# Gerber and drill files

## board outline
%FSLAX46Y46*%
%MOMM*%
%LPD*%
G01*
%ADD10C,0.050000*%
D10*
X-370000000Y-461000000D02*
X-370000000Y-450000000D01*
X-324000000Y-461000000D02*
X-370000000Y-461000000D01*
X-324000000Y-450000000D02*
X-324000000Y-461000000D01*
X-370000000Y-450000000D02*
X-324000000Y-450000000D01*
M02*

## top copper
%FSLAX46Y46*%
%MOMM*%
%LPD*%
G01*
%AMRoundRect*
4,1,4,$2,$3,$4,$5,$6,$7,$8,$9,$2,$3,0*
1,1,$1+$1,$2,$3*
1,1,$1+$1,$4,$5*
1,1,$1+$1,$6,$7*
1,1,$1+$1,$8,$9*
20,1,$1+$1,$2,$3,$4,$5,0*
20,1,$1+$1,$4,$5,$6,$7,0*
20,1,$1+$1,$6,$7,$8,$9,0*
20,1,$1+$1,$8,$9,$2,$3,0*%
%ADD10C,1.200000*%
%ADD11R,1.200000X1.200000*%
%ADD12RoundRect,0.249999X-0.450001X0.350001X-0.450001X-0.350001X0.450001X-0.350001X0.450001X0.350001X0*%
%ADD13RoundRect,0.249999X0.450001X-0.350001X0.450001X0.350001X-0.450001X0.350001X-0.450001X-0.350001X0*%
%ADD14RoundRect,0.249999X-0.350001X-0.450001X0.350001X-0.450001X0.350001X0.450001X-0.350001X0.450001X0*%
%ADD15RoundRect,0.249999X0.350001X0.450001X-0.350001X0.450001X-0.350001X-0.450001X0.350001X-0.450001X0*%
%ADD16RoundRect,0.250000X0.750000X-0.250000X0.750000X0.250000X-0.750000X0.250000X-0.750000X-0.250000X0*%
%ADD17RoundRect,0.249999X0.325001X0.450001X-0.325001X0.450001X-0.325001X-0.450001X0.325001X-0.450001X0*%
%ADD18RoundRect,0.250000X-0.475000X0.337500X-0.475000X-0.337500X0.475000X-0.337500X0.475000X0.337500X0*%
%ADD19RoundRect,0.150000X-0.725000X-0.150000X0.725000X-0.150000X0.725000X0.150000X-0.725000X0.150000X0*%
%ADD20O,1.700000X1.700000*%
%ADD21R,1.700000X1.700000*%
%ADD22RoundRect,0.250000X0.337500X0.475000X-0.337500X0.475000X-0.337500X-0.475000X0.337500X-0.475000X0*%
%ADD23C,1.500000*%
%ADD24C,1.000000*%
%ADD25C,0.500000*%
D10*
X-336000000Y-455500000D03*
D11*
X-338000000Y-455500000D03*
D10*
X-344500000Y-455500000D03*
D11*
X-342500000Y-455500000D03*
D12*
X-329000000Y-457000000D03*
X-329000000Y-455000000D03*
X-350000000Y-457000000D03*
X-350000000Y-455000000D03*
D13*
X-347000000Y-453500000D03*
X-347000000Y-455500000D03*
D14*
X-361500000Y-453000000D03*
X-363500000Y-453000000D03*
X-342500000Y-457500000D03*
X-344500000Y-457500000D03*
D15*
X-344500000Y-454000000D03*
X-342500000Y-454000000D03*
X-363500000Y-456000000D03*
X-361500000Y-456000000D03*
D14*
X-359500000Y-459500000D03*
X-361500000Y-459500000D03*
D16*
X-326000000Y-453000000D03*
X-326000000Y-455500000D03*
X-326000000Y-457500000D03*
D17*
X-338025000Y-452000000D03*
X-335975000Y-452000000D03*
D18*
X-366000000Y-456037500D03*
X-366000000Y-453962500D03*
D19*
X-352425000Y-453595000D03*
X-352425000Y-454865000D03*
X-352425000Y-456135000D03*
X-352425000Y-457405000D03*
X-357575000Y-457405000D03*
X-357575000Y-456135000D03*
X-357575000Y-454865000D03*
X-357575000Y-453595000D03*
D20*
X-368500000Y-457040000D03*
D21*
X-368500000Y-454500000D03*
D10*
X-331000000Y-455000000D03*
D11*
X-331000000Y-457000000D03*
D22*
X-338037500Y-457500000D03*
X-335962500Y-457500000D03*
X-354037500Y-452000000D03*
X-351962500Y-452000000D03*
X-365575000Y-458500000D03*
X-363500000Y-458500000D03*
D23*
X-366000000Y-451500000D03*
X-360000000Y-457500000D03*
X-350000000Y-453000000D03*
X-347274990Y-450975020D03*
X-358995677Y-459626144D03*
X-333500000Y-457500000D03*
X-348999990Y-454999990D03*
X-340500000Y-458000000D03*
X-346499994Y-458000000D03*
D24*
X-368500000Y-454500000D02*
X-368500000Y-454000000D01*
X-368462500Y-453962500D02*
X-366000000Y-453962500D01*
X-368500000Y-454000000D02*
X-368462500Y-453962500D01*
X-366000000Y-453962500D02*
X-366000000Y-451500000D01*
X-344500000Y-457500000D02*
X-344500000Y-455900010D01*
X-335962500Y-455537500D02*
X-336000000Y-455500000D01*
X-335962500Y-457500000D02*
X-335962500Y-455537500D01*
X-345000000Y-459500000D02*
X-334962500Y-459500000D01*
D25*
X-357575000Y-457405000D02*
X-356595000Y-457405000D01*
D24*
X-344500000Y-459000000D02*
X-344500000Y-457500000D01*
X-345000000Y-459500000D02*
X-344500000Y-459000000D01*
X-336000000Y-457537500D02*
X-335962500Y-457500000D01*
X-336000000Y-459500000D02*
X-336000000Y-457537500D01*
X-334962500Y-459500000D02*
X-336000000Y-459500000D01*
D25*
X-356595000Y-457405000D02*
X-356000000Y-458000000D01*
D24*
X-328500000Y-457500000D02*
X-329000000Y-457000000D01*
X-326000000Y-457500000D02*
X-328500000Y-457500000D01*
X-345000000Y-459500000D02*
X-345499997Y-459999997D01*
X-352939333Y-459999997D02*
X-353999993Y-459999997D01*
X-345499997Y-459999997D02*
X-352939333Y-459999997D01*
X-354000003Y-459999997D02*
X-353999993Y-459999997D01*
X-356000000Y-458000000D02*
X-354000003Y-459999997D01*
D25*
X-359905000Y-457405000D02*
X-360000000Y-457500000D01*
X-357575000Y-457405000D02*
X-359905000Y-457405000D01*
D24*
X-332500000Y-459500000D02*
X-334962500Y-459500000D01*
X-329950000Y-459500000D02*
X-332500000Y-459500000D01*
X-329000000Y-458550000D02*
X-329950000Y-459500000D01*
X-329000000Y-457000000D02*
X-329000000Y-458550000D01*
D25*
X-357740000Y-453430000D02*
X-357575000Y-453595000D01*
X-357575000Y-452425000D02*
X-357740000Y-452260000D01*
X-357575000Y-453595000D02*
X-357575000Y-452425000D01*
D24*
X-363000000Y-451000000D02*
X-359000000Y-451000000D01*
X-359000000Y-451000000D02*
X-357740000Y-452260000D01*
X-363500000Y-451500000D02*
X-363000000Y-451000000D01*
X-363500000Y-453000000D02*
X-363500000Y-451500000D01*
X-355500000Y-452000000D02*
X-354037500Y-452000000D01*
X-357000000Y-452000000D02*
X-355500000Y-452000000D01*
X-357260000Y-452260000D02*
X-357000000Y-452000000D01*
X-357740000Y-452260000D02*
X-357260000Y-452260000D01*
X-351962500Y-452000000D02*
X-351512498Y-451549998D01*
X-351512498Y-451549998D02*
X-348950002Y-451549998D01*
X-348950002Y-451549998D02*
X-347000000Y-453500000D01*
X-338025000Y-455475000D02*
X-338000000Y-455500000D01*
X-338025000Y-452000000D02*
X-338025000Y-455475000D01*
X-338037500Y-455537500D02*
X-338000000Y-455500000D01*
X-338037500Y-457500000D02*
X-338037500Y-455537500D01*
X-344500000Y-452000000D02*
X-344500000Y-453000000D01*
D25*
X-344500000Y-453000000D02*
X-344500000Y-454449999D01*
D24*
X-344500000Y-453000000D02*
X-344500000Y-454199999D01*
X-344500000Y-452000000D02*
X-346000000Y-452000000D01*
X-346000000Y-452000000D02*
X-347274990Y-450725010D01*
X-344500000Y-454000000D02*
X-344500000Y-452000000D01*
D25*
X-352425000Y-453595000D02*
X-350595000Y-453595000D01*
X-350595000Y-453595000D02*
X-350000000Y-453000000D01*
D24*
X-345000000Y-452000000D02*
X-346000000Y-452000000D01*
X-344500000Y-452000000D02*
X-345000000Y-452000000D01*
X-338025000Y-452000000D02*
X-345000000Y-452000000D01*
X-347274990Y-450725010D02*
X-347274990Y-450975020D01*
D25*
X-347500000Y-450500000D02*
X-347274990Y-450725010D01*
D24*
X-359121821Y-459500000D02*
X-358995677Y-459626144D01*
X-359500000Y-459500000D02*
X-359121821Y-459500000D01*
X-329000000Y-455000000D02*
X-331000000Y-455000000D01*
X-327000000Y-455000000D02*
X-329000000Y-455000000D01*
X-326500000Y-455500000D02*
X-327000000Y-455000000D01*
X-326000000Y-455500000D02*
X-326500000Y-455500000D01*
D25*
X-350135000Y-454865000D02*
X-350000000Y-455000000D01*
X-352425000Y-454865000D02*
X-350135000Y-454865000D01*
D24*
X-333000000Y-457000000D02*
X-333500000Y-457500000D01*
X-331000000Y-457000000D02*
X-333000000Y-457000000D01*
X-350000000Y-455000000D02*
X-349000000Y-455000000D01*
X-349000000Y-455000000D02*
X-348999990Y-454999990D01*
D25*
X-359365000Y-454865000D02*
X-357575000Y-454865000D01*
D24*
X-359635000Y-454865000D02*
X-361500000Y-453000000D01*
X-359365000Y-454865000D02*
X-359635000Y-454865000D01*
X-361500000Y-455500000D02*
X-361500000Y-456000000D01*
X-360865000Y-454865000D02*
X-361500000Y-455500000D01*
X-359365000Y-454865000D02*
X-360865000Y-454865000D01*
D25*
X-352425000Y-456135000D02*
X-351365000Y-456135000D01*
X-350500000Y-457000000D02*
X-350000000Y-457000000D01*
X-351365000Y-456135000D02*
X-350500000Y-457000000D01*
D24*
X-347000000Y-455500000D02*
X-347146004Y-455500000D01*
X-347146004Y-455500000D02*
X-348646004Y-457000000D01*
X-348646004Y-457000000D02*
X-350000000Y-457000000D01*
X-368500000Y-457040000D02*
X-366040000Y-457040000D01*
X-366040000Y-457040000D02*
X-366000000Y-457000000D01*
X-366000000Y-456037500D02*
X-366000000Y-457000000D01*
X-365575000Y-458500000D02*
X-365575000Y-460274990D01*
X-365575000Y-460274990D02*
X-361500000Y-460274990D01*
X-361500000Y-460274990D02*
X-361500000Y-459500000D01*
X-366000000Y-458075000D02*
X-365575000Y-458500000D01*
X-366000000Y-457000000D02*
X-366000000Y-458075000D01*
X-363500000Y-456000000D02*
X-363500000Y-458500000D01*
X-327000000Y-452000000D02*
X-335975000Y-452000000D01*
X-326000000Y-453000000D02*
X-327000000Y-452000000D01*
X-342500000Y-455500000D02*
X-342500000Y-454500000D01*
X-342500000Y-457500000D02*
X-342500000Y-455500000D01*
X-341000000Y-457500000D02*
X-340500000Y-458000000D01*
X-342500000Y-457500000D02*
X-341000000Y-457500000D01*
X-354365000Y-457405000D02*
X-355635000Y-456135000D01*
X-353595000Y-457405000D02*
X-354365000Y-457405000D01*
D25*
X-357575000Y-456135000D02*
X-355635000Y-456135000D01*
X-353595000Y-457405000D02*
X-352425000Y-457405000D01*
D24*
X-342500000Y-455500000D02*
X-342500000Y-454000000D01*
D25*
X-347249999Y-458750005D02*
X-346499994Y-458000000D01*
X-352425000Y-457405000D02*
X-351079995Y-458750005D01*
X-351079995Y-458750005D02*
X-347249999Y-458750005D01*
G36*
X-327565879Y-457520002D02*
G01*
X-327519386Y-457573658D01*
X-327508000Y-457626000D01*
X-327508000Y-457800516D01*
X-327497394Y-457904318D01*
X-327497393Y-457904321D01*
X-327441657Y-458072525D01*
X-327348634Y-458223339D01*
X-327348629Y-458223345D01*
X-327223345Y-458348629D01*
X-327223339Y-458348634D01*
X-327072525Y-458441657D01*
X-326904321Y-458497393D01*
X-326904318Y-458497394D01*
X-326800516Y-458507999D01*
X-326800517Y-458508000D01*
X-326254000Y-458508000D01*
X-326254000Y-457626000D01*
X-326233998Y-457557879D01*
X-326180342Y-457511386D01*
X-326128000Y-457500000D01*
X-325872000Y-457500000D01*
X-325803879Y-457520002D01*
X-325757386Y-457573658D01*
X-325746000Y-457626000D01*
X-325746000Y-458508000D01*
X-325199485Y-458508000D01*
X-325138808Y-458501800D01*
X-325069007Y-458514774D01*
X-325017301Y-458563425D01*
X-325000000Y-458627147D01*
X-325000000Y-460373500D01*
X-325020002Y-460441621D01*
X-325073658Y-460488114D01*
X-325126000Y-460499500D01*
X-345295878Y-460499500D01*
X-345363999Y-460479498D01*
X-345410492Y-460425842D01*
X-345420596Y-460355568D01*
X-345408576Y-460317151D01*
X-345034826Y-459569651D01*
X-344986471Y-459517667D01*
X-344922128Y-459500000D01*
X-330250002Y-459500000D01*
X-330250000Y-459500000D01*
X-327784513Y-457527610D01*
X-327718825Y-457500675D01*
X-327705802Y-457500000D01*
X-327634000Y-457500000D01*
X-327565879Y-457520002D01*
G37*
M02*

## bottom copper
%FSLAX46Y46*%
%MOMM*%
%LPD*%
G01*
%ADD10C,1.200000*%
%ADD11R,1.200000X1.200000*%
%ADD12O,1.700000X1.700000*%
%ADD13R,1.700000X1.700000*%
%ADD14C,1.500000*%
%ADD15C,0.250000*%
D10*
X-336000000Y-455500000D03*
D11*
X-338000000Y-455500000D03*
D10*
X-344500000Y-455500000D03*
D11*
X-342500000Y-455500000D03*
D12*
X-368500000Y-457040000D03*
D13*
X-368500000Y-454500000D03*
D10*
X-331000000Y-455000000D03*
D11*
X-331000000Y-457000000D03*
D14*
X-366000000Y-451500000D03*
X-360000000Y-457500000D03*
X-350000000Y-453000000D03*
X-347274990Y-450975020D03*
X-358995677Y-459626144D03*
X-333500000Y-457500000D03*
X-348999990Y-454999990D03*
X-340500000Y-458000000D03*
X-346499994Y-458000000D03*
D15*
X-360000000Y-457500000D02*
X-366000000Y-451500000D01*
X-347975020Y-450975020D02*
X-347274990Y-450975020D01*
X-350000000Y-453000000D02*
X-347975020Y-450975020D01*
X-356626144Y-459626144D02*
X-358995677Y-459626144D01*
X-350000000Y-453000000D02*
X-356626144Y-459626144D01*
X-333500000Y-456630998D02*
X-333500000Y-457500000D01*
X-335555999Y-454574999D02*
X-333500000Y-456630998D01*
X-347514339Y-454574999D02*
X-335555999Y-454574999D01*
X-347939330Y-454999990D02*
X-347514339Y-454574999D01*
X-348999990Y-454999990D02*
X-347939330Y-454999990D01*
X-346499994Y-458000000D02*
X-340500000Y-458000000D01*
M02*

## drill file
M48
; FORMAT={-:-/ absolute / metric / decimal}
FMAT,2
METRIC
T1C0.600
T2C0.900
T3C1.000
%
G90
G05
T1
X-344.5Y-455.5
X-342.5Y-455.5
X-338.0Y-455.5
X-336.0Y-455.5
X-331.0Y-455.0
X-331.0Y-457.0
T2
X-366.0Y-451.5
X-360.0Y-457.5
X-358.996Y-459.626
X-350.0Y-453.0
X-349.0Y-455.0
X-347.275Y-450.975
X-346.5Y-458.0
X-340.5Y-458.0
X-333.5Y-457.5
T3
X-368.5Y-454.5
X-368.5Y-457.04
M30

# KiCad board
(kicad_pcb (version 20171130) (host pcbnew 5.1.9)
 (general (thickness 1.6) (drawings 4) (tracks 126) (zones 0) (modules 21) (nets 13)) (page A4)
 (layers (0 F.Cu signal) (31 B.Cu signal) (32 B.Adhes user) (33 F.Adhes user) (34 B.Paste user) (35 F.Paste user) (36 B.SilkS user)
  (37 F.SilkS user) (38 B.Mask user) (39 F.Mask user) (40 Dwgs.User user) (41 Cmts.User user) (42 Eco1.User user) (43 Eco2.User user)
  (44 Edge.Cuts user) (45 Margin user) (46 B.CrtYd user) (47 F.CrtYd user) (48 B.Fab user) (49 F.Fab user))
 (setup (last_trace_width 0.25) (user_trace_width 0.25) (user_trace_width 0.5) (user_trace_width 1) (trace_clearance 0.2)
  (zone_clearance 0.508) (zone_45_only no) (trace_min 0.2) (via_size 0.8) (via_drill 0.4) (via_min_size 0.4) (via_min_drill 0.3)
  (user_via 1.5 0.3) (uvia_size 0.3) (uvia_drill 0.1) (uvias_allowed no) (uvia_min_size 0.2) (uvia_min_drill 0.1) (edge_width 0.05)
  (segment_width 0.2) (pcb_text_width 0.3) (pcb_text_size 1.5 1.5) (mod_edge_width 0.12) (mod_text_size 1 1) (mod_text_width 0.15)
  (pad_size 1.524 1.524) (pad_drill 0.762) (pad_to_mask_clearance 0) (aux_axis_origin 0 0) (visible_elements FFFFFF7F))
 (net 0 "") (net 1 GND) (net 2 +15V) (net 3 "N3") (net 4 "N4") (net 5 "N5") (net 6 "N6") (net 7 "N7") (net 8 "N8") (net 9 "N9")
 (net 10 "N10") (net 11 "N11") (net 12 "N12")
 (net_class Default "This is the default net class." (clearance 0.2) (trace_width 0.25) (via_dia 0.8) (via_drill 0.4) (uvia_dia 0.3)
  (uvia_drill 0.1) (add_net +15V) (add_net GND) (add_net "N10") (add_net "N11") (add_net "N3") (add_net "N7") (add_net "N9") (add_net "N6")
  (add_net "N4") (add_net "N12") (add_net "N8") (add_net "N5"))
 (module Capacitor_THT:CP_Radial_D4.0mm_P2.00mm (layer B.Cu) (at -338 455.5)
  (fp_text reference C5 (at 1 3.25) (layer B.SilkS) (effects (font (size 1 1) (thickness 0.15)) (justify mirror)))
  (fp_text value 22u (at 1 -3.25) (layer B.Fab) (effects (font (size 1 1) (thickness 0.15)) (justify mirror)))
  (pad 2 thru_hole circle (at 2 0) (size 1.2 1.2) (drill 0.6) (layers *.Cu *.Mask) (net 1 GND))
  (pad 1 thru_hole rect (at 0 0) (size 1.2 1.2) (drill 0.6) (layers *.Cu *.Mask) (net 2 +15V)))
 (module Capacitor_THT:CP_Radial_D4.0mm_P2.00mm (layer B.Cu) (at -342.5 455.5 180)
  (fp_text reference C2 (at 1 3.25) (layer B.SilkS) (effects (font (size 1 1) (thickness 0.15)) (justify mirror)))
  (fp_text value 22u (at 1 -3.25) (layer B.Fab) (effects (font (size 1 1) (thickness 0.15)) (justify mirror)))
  (pad 2 thru_hole circle (at 2 0 180) (size 1.2 1.2) (drill 0.6) (layers *.Cu *.Mask) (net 1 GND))
  (pad 1 thru_hole rect (at 0 0 180) (size 1.2 1.2) (drill 0.6) (layers *.Cu *.Mask) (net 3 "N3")))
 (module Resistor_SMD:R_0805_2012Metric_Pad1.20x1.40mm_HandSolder (layer F.Cu) (at -329 456 270)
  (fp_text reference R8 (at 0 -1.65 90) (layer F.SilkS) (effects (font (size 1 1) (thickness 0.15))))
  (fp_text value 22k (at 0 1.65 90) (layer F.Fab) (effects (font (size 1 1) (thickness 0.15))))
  (pad 2 smd roundrect (at 1 0 270) (size 1.2 1.4) (layers F.Cu F.Paste F.Mask) (roundrect_rratio 0.2083325) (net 1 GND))
  (pad 1 smd roundrect (at -1 0 270) (size 1.2 1.4) (layers F.Cu F.Paste F.Mask) (roundrect_rratio 0.2083325) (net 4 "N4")))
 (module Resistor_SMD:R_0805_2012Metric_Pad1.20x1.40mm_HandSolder (layer F.Cu) (at -350 456 270)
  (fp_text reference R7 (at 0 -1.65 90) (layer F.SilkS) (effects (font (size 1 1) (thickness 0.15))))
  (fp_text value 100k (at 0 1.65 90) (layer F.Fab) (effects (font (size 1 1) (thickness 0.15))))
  (pad 2 smd roundrect (at 1 0 270) (size 1.2 1.4) (layers F.Cu F.Paste F.Mask) (roundrect_rratio 0.2083325) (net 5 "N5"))
  (pad 1 smd roundrect (at -1 0 270) (size 1.2 1.4) (layers F.Cu F.Paste F.Mask) (roundrect_rratio 0.2083325) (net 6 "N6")))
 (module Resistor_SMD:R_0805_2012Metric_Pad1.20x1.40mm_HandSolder (layer F.Cu) (at -347 454.5 90)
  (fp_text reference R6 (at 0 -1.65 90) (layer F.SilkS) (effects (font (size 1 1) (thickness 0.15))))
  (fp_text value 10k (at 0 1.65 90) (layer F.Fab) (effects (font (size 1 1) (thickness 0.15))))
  (pad 2 smd roundrect (at 1 0 90) (size 1.2 1.4) (layers F.Cu F.Paste F.Mask) (roundrect_rratio 0.2083325) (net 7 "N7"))
  (pad 1 smd roundrect (at -1 0 90) (size 1.2 1.4) (layers F.Cu F.Paste F.Mask) (roundrect_rratio 0.2083325) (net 5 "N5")))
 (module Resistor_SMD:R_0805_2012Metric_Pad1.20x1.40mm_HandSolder (layer F.Cu) (at -362.5 453)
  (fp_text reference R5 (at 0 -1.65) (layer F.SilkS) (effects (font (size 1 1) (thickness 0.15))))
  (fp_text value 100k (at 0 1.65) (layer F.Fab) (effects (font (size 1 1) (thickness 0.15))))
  (pad 2 smd roundrect (at 1 0) (size 1.2 1.4) (layers F.Cu F.Paste F.Mask) (roundrect_rratio 0.2083325) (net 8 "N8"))
  (pad 1 smd roundrect (at -1 0) (size 1.2 1.4) (layers F.Cu F.Paste F.Mask) (roundrect_rratio 0.2083325) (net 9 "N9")))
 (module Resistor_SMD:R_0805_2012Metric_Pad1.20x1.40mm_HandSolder (layer F.Cu) (at -343.5 457.5)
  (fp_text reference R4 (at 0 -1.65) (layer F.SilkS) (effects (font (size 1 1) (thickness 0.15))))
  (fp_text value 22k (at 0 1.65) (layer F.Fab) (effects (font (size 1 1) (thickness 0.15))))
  (pad 2 smd roundrect (at 1 0) (size 1.2 1.4) (layers F.Cu F.Paste F.Mask) (roundrect_rratio 0.2083325) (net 3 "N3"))
  (pad 1 smd roundrect (at -1 0) (size 1.2 1.4) (layers F.Cu F.Paste F.Mask) (roundrect_rratio 0.2083325) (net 1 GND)))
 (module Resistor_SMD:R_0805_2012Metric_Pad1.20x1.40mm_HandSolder (layer F.Cu) (at -343.5 454 180)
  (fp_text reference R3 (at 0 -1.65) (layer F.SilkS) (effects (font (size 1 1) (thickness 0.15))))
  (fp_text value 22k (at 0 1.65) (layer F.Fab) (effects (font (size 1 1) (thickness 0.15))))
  (pad 2 smd roundrect (at 1 0 180) (size 1.2 1.4) (layers F.Cu F.Paste F.Mask) (roundrect_rratio 0.2083325) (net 2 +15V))
  (pad 1 smd roundrect (at -1 0 180) (size 1.2 1.4) (layers F.Cu F.Paste F.Mask) (roundrect_rratio 0.2083325) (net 3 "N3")))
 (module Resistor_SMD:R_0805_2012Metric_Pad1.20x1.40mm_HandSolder (layer F.Cu) (at -362.5 456 180)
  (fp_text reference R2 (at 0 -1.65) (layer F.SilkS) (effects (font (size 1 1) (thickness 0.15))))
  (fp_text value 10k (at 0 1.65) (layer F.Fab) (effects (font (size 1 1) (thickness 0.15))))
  (pad 2 smd roundrect (at 1 0 180) (size 1.2 1.4) (layers F.Cu F.Paste F.Mask) (roundrect_rratio 0.2083325) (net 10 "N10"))
  (pad 1 smd roundrect (at -1 0 180) (size 1.2 1.4) (layers F.Cu F.Paste F.Mask) (roundrect_rratio 0.2083325) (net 8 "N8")))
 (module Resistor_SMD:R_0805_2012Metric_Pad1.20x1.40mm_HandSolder (layer F.Cu) (at -360.5 459.5)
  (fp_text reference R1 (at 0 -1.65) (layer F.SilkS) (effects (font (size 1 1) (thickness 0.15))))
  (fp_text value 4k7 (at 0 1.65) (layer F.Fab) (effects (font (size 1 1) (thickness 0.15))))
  (pad 2 smd roundrect (at 1 0) (size 1.2 1.4) (layers F.Cu F.Paste F.Mask) (roundrect_rratio 0.2083325) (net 2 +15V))
  (pad 1 smd roundrect (at -1 0) (size 1.2 1.4) (layers F.Cu F.Paste F.Mask) (roundrect_rratio 0.2083325) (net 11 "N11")))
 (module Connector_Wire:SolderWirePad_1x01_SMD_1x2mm (layer F.Cu) (at -326 453 90)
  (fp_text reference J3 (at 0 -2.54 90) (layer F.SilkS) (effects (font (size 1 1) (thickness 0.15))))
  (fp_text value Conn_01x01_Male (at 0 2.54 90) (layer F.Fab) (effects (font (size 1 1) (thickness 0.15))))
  (pad 1 smd roundrect (at 0 0 90) (size 1 2) (layers F.Cu F.Paste F.Mask) (roundrect_rratio 0.25) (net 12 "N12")))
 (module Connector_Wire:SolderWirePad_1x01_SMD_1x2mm (layer F.Cu) (at -326 455.5 90)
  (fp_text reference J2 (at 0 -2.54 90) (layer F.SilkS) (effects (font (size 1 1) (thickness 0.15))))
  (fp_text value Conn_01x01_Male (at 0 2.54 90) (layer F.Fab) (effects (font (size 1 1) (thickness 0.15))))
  (pad 1 smd roundrect (at 0 0 90) (size 1 2) (layers F.Cu F.Paste F.Mask) (roundrect_rratio 0.25) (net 4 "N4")))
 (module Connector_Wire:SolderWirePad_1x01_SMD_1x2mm (layer F.Cu) (at -326 457.5 90)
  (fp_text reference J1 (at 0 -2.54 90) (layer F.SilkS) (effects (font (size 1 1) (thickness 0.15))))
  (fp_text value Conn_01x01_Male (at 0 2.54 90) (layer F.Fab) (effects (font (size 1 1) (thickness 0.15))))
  (pad 1 smd roundrect (at 0 0 90) (size 1 2) (layers F.Cu F.Paste F.Mask) (roundrect_rratio 0.25) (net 1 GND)))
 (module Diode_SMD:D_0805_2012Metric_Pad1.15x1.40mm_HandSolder (layer F.Cu) (at -337 452 180)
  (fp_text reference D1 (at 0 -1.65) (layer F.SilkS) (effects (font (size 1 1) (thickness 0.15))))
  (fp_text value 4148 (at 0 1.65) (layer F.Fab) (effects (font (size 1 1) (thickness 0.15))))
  (pad 2 smd roundrect (at 1.025 0 180) (size 1.15 1.4) (layers F.Cu F.Paste F.Mask) (roundrect_rratio 0.2173904347826087) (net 2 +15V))
  (pad 1 smd roundrect (at -1.025 0 180) (size 1.15 1.4) (layers F.Cu F.Paste F.Mask) (roundrect_rratio 0.2173904347826087) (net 12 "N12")))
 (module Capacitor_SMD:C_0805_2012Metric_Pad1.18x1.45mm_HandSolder (layer F.Cu) (at -366 455 270)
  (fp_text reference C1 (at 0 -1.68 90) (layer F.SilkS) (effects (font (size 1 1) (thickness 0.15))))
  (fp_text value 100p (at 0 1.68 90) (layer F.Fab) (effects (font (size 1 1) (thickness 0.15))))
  (pad 2 smd roundrect (at 1.0375 0 270) (size 1.175 1.45) (layers F.Cu F.Paste F.Mask) (roundrect_rratio 0.2127659574468085) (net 11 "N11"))
  (pad 1 smd roundrect (at -1.0375 0 270) (size 1.175 1.45) (layers F.Cu F.Paste F.Mask) (roundrect_rratio 0.2127659574468085) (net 1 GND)))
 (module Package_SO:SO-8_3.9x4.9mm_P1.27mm (layer F.Cu) (at -355 455.5)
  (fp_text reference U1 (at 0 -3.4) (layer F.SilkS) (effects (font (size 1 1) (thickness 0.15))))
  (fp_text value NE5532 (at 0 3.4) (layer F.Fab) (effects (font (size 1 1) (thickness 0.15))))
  (pad 8 smd roundrect (at 2.575 -1.905) (size 1.75 0.6) (layers F.Cu F.Paste F.Mask) (roundrect_rratio 0.25) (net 2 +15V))
  (pad 7 smd roundrect (at 2.575 -0.635) (size 1.75 0.6) (layers F.Cu F.Paste F.Mask) (roundrect_rratio 0.25) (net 6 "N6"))
  (pad 6 smd roundrect (at 2.575 0.635) (size 1.75 0.6) (layers F.Cu F.Paste F.Mask) (roundrect_rratio 0.25) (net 5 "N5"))
  (pad 5 smd roundrect (at 2.575 1.905) (size 1.75 0.6) (layers F.Cu F.Paste F.Mask) (roundrect_rratio 0.25) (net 3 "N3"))
  (pad 4 smd roundrect (at -2.575 1.905) (size 1.75 0.6) (layers F.Cu F.Paste F.Mask) (roundrect_rratio 0.25) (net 1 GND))
  (pad 3 smd roundrect (at -2.575 0.635) (size 1.75 0.6) (layers F.Cu F.Paste F.Mask) (roundrect_rratio 0.25) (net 3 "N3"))
  (pad 2 smd roundrect (at -2.575 -0.635) (size 1.75 0.6) (layers F.Cu F.Paste F.Mask) (roundrect_rratio 0.25) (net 8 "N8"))
  (pad 1 smd roundrect (at -2.575 -1.905) (size 1.75 0.6) (layers F.Cu F.Paste F.Mask) (roundrect_rratio 0.25) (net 9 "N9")))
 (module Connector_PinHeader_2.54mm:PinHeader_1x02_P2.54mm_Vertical (layer B.Cu) (at -368.5 454.5 180)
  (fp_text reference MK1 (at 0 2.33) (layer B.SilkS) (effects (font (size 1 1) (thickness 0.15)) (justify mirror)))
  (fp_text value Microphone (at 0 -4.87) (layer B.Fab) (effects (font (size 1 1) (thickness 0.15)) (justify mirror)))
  (pad 2 thru_hole oval (at 0 -2.54 180) (size 1.7 1.7) (drill 1) (layers *.Cu *.Mask) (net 11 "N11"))
  (pad 1 thru_hole rect (at 0 0 180) (size 1.7 1.7) (drill 1) (layers *.Cu *.Mask) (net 1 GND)))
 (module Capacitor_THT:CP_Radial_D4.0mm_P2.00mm (layer B.Cu) (at -331 457 90)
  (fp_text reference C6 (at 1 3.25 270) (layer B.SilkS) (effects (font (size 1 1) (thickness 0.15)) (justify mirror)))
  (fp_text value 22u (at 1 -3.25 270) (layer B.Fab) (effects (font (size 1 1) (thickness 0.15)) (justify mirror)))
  (pad 2 thru_hole circle (at 2 0 90) (size 1.2 1.2) (drill 0.6) (layers *.Cu *.Mask) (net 4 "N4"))
  (pad 1 thru_hole rect (at 0 0 90) (size 1.2 1.2) (drill 0.6) (layers *.Cu *.Mask) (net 6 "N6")))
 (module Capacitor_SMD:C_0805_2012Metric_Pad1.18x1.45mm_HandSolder (layer F.Cu) (at -337 457.5 180)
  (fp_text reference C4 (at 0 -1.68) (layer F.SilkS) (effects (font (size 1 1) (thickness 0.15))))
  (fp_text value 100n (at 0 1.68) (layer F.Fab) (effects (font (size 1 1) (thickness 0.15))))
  (pad 2 smd roundrect (at 1.0375 0 180) (size 1.175 1.45) (layers F.Cu F.Paste F.Mask) (roundrect_rratio 0.2127659574468085) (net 2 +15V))
  (pad 1 smd roundrect (at -1.0375 0 180) (size 1.175 1.45) (layers F.Cu F.Paste F.Mask) (roundrect_rratio 0.2127659574468085) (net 1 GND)))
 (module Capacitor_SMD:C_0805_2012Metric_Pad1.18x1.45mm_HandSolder (layer F.Cu) (at -353 452 180)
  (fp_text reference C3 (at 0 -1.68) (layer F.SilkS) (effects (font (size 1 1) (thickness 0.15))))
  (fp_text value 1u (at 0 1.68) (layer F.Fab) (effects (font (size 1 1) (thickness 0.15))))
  (pad 2 smd roundrect (at 1.0375 0 180) (size 1.175 1.45) (layers F.Cu F.Paste F.Mask) (roundrect_rratio 0.2127659574468085) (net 9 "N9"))
  (pad 1 smd roundrect (at -1.0375 0 180) (size 1.175 1.45) (layers F.Cu F.Paste F.Mask) (roundrect_rratio 0.2127659574468085) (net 7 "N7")))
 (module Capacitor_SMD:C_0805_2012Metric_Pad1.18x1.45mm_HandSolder (layer F.Cu) (at -364.5375 458.5 180)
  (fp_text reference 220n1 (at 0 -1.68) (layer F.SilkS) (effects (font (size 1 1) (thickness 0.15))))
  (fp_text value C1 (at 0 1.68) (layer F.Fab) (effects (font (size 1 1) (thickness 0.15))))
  (pad 2 smd roundrect (at 1.0375 0 180) (size 1.175 1.45) (layers F.Cu F.Paste F.Mask) (roundrect_rratio 0.2127659574468085) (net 11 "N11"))
  (pad 1 smd roundrect (at -1.0375 0 180) (size 1.175 1.45) (layers F.Cu F.Paste F.Mask) (roundrect_rratio 0.2127659574468085)
   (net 10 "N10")))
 (gr_line (start -370 461) (end -370 450) (layer Edge.Cuts) (width 0.05))
 (gr_line (start -324 461) (end -370 461) (layer Edge.Cuts) (width 0.05))
 (gr_line (start -324 450) (end -324 461) (layer Edge.Cuts) (width 0.05))
 (gr_line (start -370 450) (end -324 450) (layer Edge.Cuts) (width 0.05))
 (segment (start -368.5 454.5) (end -368.5 454) (width 1) (layer F.Cu) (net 1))
 (segment (start -368.4625 453.9625) (end -366 453.9625) (width 1) (layer F.Cu) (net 1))
 (segment (start -368.5 454) (end -368.4625 453.9625) (width 1) (layer F.Cu) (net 1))
 (via (at -366 451.5) (size 1.5) (drill 0.9) (layers F.Cu B.Cu) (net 1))
 (segment (start -366 453.9625) (end -366 451.5) (width 1) (layer F.Cu) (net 1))
 (segment (start -344.5 457.5) (end -344.5 455.90001) (width 1) (layer F.Cu) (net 1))
 (segment (start -335.9625 455.5375) (end -336 455.5) (width 1) (layer F.Cu) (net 1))
 (segment (start -335.9625 457.5) (end -335.9625 455.5375) (width 1) (layer F.Cu) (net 1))
 (segment (start -345 459.5) (end -334.9625 459.5) (width 1) (layer F.Cu) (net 1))
 (segment (start -357.575 457.405) (end -356.595 457.405) (width 0.5) (layer F.Cu) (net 1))
 (segment (start -344.5 459) (end -344.5 457.5) (width 1) (layer F.Cu) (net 1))
 (segment (start -345 459.5) (end -344.5 459) (width 1) (layer F.Cu) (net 1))
 (segment (start -336 457.5375) (end -335.9625 457.5) (width 1) (layer F.Cu) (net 1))
 (segment (start -336 459.5) (end -336 457.5375) (width 1) (layer F.Cu) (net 1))
 (segment (start -334.9625 459.5) (end -336 459.5) (width 1) (layer F.Cu) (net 1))
 (segment (start -356.595 457.405) (end -356 458) (width 0.5) (layer F.Cu) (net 1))
 (segment (start -328.5 457.5) (end -329 457) (width 1) (layer F.Cu) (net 1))
 (segment (start -326 457.5) (end -328.5 457.5) (width 1) (layer F.Cu) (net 1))
 (segment (start -345 459.5) (end -345.499997 459.999997) (width 1) (layer F.Cu) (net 1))
 (segment (start -352.939333 459.999997) (end -353.999993 459.999997) (width 1) (layer F.Cu) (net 1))
 (segment (start -345.499997 459.999997) (end -352.939333 459.999997) (width 1) (layer F.Cu) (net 1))
 (segment (start -354.000003 459.999997) (end -353.999993 459.999997) (width 1) (layer F.Cu) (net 1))
 (segment (start -356 458) (end -354.000003 459.999997) (width 1) (layer F.Cu) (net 1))
 (via (at -360 457.5) (size 1.5) (drill 0.9) (layers F.Cu B.Cu) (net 1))
 (segment (start -359.905 457.405) (end -360 457.5) (width 0.5) (layer F.Cu) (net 1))
 (segment (start -357.575 457.405) (end -359.905 457.405) (width 0.5) (layer F.Cu) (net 1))
 (segment (start -360 457.5) (end -366 451.5) (width 0.25) (layer B.Cu) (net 1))
 (segment (start -332.5 459.5) (end -334.9625 459.5) (width 1) (layer F.Cu) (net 1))
 (segment (start -329.95 459.5) (end -332.5 459.5) (width 1) (layer F.Cu) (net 1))
 (segment (start -329 458.55) (end -329.95 459.5) (width 1) (layer F.Cu) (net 1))
 (segment (start -329 457) (end -329 458.55) (width 1) (layer F.Cu) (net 1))
 (segment (start -357.74 453.43) (end -357.575 453.595) (width 0.5) (layer F.Cu) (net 9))
 (segment (start -357.575 452.425) (end -357.74 452.26) (width 0.5) (layer F.Cu) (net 9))
 (segment (start -357.575 453.595) (end -357.575 452.425) (width 0.5) (layer F.Cu) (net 9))
 (segment (start -363 451) (end -359 451) (width 1) (layer F.Cu) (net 9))
 (segment (start -359 451) (end -357.74 452.26) (width 1) (layer F.Cu) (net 9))
 (segment (start -363.5 451.5) (end -363 451) (width 1) (layer F.Cu) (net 9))
 (segment (start -363.5 453) (end -363.5 451.5) (width 1) (layer F.Cu) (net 9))
 (segment (start -355.5 452) (end -354.0375 452) (width 1) (layer F.Cu) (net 9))
 (segment (start -357 452) (end -355.5 452) (width 1) (layer F.Cu) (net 9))
 (segment (start -357.26 452.26) (end -357 452) (width 1) (layer F.Cu) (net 9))
 (segment (start -357.74 452.26) (end -357.26 452.26) (width 1) (layer F.Cu) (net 9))
 (segment (start -351.9625 452) (end -351.512498 451.549998) (width 1) (layer F.Cu) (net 7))
 (segment (start -351.512498 451.549998) (end -348.950002 451.549998) (width 1) (layer F.Cu) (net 7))
 (segment (start -348.950002 451.549998) (end -347 453.5) (width 1) (layer F.Cu) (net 7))
 (segment (start -338.025 455.475) (end -338 455.5) (width 1) (layer F.Cu) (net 2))
 (segment (start -338.025 452) (end -338.025 455.475) (width 1) (layer F.Cu) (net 2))
 (segment (start -338.0375 455.5375) (end -338 455.5) (width 1) (layer F.Cu) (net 2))
 (segment (start -338.0375 457.5) (end -338.0375 455.5375) (width 1) (layer F.Cu) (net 2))
 (segment (start -344.5 452) (end -344.5 453) (width 1) (layer F.Cu) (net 2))
 (segment (start -344.5 453) (end -344.5 454.449999) (width 0.5) (layer F.Cu) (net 2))
 (segment (start -344.5 453) (end -344.5 454.199999) (width 1) (layer F.Cu) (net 2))
 (segment (start -344.5 452) (end -346 452) (width 1) (layer F.Cu) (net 2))
 (segment (start -346 452) (end -347.27499 450.72501) (width 1) (layer F.Cu) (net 2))
 (segment (start -344.5 454) (end -344.5 452) (width 1) (layer F.Cu) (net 2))
 (via (at -350 453) (size 1.5) (drill 0.9) (layers F.Cu B.Cu) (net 2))
 (segment (start -352.425 453.595) (end -350.595 453.595) (width 0.5) (layer F.Cu) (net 2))
 (segment (start -350.595 453.595) (end -350 453) (width 0.5) (layer F.Cu) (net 2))
 (segment (start -345 452) (end -346 452) (width 1) (layer F.Cu) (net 2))
 (segment (start -344.5 452) (end -345 452) (width 1) (layer F.Cu) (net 2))
 (segment (start -338.025 452) (end -345 452) (width 1) (layer F.Cu) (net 2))
 (segment (start -347.27499 450.72501) (end -347.27499 450.97502) (width 1) (layer F.Cu) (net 2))
 (segment (start -347.5 450.5) (end -347.27499 450.72501) (width 0.5) (layer F.Cu) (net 2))
 (via (at -347.27499 450.97502) (size 1.5) (drill 0.9) (layers F.Cu B.Cu) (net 2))
 (segment (start -347.97502 450.97502) (end -347.27499 450.97502) (width 0.25) (layer B.Cu) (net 2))
 (segment (start -350 453) (end -347.97502 450.97502) (width 0.25) (layer B.Cu) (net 2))
 (segment (start -356.626144 459.626144) (end -358.995677 459.626144) (width 0.25) (layer B.Cu) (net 2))
 (segment (start -350 453) (end -356.626144 459.626144) (width 0.25) (layer B.Cu) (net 2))
 (via (at -358.995677 459.626144) (size 1.5) (drill 0.9) (layers F.Cu B.Cu) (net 2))
 (segment (start -359.121821 459.5) (end -358.995677 459.626144) (width 1) (layer F.Cu) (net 2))
 (segment (start -359.5 459.5) (end -359.121821 459.5) (width 1) (layer F.Cu) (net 2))
 (segment (start -329 455) (end -331 455) (width 1) (layer F.Cu) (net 4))
 (segment (start -327 455) (end -329 455) (width 1) (layer F.Cu) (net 4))
 (segment (start -326.5 455.5) (end -327 455) (width 1) (layer F.Cu) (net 4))
 (segment (start -326 455.5) (end -326.5 455.5) (width 1) (layer F.Cu) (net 4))
 (segment (start -350.135 454.865) (end -350 455) (width 0.5) (layer F.Cu) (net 6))
 (segment (start -352.425 454.865) (end -350.135 454.865) (width 0.5) (layer F.Cu) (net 6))
 (via (at -333.5 457.5) (size 1.5) (drill 0.9) (layers F.Cu B.Cu) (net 6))
 (segment (start -333 457) (end -333.5 457.5) (width 1) (layer F.Cu) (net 6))
 (segment (start -331 457) (end -333 457) (width 1) (layer F.Cu) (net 6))
 (via (at -348.99999 454.99999) (size 1.5) (drill 0.9) (layers F.Cu B.Cu) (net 6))
 (segment (start -350 455) (end -349 455) (width 1) (layer F.Cu) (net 6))
 (segment (start -349 455) (end -348.99999 454.99999) (width 1) (layer F.Cu) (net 6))
 (segment (start -333.5 456.630998) (end -333.5 457.5) (width 0.25) (layer B.Cu) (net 6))
 (segment (start -335.555999 454.574999) (end -333.5 456.630998) (width 0.25) (layer B.Cu) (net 6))
 (segment (start -347.514339 454.574999) (end -335.555999 454.574999) (width 0.25) (layer B.Cu) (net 6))
 (segment (start -347.93933 454.99999) (end -347.514339 454.574999) (width 0.25) (layer B.Cu) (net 6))
 (segment (start -348.99999 454.99999) (end -347.93933 454.99999) (width 0.25) (layer B.Cu) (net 6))
 (segment (start -359.365 454.865) (end -357.575 454.865) (width 0.5) (layer F.Cu) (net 8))
 (segment (start -359.635 454.865) (end -361.5 453) (width 1) (layer F.Cu) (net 8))
 (segment (start -359.365 454.865) (end -359.635 454.865) (width 1) (layer F.Cu) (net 8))
 (segment (start -361.5 455.5) (end -361.5 456) (width 1) (layer F.Cu) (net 8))
 (segment (start -360.865 454.865) (end -361.5 455.5) (width 1) (layer F.Cu) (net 8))
 (segment (start -359.365 454.865) (end -360.865 454.865) (width 1) (layer F.Cu) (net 8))
 (segment (start -352.425 456.135) (end -351.365 456.135) (width 0.5) (layer F.Cu) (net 5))
 (segment (start -350.5 457) (end -350 457) (width 0.5) (layer F.Cu) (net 5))
 (segment (start -351.365 456.135) (end -350.5 457) (width 0.5) (layer F.Cu) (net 5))
 (segment (start -347 455.5) (end -347.146004 455.5) (width 1) (layer F.Cu) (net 5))
 (segment (start -347.146004 455.5) (end -348.646004 457) (width 1) (layer F.Cu) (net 5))
 (segment (start -348.646004 457) (end -350 457) (width 1) (layer F.Cu) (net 5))
 (segment (start -368.5 457.04) (end -366.04 457.04) (width 1) (layer F.Cu) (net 11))
 (segment (start -366.04 457.04) (end -366 457) (width 1) (layer F.Cu) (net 11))
 (segment (start -366 456.0375) (end -366 457) (width 1) (layer F.Cu) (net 11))
 (segment (start -365.575 458.5) (end -365.575 460.27499) (width 1) (layer F.Cu) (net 11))
 (segment (start -365.575 460.27499) (end -361.5 460.27499) (width 1) (layer F.Cu) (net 11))
 (segment (start -361.5 460.27499) (end -361.5 459.5) (width 1) (layer F.Cu) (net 11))
 (segment (start -366 458.075) (end -365.575 458.5) (width 1) (layer F.Cu) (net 11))
 (segment (start -366 457) (end -366 458.075) (width 1) (layer F.Cu) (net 11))
 (segment (start -363.5 456) (end -363.5 458.5) (width 1) (layer F.Cu) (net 10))
 (segment (start -327 452) (end -335.975 452) (width 1) (layer F.Cu) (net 12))
 (segment (start -326 453) (end -327 452) (width 1) (layer F.Cu) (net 12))
 (segment (start -342.5 455.5) (end -342.5 454.5) (width 1) (layer F.Cu) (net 3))
 (segment (start -342.5 457.5) (end -342.5 455.5) (width 1) (layer F.Cu) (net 3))
 (via (at -340.5 458) (size 1.5) (drill 0.9) (layers F.Cu B.Cu) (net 3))
 (segment (start -341 457.5) (end -340.5 458) (width 1) (layer F.Cu) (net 3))
 (segment (start -342.5 457.5) (end -341 457.5) (width 1) (layer F.Cu) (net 3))
 (segment (start -354.365 457.405) (end -355.635 456.135) (width 1) (layer F.Cu) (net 3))
 (segment (start -353.595 457.405) (end -354.365 457.405) (width 1) (layer F.Cu) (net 3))
 (segment (start -357.575 456.135) (end -355.635 456.135) (width 0.5) (layer F.Cu) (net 3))
 (segment (start -353.595 457.405) (end -352.425 457.405) (width 0.5) (layer F.Cu) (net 3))
 (segment (start -342.5 455.5) (end -342.5 454) (width 1) (layer F.Cu) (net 3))
 (via (at -346.499994 458) (size 1.5) (drill 0.9) (layers F.Cu B.Cu) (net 3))
 (segment (start -347.249999 458.750005) (end -346.499994 458) (width 0.5) (layer F.Cu) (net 3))
 (segment (start -352.425 457.405) (end -351.079995 458.750005) (width 0.5) (layer F.Cu) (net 3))
 (segment (start -351.079995 458.750005) (end -347.249999 458.750005) (width 0.5) (layer F.Cu) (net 3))
 (segment (start -346.499994 458) (end -340.5 458) (width 0.25) (layer B.Cu) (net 3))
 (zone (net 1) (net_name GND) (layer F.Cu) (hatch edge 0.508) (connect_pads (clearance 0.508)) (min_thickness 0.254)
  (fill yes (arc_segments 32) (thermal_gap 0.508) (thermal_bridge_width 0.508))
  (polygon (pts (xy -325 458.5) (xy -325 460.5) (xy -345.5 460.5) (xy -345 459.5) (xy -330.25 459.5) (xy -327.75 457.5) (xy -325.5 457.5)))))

